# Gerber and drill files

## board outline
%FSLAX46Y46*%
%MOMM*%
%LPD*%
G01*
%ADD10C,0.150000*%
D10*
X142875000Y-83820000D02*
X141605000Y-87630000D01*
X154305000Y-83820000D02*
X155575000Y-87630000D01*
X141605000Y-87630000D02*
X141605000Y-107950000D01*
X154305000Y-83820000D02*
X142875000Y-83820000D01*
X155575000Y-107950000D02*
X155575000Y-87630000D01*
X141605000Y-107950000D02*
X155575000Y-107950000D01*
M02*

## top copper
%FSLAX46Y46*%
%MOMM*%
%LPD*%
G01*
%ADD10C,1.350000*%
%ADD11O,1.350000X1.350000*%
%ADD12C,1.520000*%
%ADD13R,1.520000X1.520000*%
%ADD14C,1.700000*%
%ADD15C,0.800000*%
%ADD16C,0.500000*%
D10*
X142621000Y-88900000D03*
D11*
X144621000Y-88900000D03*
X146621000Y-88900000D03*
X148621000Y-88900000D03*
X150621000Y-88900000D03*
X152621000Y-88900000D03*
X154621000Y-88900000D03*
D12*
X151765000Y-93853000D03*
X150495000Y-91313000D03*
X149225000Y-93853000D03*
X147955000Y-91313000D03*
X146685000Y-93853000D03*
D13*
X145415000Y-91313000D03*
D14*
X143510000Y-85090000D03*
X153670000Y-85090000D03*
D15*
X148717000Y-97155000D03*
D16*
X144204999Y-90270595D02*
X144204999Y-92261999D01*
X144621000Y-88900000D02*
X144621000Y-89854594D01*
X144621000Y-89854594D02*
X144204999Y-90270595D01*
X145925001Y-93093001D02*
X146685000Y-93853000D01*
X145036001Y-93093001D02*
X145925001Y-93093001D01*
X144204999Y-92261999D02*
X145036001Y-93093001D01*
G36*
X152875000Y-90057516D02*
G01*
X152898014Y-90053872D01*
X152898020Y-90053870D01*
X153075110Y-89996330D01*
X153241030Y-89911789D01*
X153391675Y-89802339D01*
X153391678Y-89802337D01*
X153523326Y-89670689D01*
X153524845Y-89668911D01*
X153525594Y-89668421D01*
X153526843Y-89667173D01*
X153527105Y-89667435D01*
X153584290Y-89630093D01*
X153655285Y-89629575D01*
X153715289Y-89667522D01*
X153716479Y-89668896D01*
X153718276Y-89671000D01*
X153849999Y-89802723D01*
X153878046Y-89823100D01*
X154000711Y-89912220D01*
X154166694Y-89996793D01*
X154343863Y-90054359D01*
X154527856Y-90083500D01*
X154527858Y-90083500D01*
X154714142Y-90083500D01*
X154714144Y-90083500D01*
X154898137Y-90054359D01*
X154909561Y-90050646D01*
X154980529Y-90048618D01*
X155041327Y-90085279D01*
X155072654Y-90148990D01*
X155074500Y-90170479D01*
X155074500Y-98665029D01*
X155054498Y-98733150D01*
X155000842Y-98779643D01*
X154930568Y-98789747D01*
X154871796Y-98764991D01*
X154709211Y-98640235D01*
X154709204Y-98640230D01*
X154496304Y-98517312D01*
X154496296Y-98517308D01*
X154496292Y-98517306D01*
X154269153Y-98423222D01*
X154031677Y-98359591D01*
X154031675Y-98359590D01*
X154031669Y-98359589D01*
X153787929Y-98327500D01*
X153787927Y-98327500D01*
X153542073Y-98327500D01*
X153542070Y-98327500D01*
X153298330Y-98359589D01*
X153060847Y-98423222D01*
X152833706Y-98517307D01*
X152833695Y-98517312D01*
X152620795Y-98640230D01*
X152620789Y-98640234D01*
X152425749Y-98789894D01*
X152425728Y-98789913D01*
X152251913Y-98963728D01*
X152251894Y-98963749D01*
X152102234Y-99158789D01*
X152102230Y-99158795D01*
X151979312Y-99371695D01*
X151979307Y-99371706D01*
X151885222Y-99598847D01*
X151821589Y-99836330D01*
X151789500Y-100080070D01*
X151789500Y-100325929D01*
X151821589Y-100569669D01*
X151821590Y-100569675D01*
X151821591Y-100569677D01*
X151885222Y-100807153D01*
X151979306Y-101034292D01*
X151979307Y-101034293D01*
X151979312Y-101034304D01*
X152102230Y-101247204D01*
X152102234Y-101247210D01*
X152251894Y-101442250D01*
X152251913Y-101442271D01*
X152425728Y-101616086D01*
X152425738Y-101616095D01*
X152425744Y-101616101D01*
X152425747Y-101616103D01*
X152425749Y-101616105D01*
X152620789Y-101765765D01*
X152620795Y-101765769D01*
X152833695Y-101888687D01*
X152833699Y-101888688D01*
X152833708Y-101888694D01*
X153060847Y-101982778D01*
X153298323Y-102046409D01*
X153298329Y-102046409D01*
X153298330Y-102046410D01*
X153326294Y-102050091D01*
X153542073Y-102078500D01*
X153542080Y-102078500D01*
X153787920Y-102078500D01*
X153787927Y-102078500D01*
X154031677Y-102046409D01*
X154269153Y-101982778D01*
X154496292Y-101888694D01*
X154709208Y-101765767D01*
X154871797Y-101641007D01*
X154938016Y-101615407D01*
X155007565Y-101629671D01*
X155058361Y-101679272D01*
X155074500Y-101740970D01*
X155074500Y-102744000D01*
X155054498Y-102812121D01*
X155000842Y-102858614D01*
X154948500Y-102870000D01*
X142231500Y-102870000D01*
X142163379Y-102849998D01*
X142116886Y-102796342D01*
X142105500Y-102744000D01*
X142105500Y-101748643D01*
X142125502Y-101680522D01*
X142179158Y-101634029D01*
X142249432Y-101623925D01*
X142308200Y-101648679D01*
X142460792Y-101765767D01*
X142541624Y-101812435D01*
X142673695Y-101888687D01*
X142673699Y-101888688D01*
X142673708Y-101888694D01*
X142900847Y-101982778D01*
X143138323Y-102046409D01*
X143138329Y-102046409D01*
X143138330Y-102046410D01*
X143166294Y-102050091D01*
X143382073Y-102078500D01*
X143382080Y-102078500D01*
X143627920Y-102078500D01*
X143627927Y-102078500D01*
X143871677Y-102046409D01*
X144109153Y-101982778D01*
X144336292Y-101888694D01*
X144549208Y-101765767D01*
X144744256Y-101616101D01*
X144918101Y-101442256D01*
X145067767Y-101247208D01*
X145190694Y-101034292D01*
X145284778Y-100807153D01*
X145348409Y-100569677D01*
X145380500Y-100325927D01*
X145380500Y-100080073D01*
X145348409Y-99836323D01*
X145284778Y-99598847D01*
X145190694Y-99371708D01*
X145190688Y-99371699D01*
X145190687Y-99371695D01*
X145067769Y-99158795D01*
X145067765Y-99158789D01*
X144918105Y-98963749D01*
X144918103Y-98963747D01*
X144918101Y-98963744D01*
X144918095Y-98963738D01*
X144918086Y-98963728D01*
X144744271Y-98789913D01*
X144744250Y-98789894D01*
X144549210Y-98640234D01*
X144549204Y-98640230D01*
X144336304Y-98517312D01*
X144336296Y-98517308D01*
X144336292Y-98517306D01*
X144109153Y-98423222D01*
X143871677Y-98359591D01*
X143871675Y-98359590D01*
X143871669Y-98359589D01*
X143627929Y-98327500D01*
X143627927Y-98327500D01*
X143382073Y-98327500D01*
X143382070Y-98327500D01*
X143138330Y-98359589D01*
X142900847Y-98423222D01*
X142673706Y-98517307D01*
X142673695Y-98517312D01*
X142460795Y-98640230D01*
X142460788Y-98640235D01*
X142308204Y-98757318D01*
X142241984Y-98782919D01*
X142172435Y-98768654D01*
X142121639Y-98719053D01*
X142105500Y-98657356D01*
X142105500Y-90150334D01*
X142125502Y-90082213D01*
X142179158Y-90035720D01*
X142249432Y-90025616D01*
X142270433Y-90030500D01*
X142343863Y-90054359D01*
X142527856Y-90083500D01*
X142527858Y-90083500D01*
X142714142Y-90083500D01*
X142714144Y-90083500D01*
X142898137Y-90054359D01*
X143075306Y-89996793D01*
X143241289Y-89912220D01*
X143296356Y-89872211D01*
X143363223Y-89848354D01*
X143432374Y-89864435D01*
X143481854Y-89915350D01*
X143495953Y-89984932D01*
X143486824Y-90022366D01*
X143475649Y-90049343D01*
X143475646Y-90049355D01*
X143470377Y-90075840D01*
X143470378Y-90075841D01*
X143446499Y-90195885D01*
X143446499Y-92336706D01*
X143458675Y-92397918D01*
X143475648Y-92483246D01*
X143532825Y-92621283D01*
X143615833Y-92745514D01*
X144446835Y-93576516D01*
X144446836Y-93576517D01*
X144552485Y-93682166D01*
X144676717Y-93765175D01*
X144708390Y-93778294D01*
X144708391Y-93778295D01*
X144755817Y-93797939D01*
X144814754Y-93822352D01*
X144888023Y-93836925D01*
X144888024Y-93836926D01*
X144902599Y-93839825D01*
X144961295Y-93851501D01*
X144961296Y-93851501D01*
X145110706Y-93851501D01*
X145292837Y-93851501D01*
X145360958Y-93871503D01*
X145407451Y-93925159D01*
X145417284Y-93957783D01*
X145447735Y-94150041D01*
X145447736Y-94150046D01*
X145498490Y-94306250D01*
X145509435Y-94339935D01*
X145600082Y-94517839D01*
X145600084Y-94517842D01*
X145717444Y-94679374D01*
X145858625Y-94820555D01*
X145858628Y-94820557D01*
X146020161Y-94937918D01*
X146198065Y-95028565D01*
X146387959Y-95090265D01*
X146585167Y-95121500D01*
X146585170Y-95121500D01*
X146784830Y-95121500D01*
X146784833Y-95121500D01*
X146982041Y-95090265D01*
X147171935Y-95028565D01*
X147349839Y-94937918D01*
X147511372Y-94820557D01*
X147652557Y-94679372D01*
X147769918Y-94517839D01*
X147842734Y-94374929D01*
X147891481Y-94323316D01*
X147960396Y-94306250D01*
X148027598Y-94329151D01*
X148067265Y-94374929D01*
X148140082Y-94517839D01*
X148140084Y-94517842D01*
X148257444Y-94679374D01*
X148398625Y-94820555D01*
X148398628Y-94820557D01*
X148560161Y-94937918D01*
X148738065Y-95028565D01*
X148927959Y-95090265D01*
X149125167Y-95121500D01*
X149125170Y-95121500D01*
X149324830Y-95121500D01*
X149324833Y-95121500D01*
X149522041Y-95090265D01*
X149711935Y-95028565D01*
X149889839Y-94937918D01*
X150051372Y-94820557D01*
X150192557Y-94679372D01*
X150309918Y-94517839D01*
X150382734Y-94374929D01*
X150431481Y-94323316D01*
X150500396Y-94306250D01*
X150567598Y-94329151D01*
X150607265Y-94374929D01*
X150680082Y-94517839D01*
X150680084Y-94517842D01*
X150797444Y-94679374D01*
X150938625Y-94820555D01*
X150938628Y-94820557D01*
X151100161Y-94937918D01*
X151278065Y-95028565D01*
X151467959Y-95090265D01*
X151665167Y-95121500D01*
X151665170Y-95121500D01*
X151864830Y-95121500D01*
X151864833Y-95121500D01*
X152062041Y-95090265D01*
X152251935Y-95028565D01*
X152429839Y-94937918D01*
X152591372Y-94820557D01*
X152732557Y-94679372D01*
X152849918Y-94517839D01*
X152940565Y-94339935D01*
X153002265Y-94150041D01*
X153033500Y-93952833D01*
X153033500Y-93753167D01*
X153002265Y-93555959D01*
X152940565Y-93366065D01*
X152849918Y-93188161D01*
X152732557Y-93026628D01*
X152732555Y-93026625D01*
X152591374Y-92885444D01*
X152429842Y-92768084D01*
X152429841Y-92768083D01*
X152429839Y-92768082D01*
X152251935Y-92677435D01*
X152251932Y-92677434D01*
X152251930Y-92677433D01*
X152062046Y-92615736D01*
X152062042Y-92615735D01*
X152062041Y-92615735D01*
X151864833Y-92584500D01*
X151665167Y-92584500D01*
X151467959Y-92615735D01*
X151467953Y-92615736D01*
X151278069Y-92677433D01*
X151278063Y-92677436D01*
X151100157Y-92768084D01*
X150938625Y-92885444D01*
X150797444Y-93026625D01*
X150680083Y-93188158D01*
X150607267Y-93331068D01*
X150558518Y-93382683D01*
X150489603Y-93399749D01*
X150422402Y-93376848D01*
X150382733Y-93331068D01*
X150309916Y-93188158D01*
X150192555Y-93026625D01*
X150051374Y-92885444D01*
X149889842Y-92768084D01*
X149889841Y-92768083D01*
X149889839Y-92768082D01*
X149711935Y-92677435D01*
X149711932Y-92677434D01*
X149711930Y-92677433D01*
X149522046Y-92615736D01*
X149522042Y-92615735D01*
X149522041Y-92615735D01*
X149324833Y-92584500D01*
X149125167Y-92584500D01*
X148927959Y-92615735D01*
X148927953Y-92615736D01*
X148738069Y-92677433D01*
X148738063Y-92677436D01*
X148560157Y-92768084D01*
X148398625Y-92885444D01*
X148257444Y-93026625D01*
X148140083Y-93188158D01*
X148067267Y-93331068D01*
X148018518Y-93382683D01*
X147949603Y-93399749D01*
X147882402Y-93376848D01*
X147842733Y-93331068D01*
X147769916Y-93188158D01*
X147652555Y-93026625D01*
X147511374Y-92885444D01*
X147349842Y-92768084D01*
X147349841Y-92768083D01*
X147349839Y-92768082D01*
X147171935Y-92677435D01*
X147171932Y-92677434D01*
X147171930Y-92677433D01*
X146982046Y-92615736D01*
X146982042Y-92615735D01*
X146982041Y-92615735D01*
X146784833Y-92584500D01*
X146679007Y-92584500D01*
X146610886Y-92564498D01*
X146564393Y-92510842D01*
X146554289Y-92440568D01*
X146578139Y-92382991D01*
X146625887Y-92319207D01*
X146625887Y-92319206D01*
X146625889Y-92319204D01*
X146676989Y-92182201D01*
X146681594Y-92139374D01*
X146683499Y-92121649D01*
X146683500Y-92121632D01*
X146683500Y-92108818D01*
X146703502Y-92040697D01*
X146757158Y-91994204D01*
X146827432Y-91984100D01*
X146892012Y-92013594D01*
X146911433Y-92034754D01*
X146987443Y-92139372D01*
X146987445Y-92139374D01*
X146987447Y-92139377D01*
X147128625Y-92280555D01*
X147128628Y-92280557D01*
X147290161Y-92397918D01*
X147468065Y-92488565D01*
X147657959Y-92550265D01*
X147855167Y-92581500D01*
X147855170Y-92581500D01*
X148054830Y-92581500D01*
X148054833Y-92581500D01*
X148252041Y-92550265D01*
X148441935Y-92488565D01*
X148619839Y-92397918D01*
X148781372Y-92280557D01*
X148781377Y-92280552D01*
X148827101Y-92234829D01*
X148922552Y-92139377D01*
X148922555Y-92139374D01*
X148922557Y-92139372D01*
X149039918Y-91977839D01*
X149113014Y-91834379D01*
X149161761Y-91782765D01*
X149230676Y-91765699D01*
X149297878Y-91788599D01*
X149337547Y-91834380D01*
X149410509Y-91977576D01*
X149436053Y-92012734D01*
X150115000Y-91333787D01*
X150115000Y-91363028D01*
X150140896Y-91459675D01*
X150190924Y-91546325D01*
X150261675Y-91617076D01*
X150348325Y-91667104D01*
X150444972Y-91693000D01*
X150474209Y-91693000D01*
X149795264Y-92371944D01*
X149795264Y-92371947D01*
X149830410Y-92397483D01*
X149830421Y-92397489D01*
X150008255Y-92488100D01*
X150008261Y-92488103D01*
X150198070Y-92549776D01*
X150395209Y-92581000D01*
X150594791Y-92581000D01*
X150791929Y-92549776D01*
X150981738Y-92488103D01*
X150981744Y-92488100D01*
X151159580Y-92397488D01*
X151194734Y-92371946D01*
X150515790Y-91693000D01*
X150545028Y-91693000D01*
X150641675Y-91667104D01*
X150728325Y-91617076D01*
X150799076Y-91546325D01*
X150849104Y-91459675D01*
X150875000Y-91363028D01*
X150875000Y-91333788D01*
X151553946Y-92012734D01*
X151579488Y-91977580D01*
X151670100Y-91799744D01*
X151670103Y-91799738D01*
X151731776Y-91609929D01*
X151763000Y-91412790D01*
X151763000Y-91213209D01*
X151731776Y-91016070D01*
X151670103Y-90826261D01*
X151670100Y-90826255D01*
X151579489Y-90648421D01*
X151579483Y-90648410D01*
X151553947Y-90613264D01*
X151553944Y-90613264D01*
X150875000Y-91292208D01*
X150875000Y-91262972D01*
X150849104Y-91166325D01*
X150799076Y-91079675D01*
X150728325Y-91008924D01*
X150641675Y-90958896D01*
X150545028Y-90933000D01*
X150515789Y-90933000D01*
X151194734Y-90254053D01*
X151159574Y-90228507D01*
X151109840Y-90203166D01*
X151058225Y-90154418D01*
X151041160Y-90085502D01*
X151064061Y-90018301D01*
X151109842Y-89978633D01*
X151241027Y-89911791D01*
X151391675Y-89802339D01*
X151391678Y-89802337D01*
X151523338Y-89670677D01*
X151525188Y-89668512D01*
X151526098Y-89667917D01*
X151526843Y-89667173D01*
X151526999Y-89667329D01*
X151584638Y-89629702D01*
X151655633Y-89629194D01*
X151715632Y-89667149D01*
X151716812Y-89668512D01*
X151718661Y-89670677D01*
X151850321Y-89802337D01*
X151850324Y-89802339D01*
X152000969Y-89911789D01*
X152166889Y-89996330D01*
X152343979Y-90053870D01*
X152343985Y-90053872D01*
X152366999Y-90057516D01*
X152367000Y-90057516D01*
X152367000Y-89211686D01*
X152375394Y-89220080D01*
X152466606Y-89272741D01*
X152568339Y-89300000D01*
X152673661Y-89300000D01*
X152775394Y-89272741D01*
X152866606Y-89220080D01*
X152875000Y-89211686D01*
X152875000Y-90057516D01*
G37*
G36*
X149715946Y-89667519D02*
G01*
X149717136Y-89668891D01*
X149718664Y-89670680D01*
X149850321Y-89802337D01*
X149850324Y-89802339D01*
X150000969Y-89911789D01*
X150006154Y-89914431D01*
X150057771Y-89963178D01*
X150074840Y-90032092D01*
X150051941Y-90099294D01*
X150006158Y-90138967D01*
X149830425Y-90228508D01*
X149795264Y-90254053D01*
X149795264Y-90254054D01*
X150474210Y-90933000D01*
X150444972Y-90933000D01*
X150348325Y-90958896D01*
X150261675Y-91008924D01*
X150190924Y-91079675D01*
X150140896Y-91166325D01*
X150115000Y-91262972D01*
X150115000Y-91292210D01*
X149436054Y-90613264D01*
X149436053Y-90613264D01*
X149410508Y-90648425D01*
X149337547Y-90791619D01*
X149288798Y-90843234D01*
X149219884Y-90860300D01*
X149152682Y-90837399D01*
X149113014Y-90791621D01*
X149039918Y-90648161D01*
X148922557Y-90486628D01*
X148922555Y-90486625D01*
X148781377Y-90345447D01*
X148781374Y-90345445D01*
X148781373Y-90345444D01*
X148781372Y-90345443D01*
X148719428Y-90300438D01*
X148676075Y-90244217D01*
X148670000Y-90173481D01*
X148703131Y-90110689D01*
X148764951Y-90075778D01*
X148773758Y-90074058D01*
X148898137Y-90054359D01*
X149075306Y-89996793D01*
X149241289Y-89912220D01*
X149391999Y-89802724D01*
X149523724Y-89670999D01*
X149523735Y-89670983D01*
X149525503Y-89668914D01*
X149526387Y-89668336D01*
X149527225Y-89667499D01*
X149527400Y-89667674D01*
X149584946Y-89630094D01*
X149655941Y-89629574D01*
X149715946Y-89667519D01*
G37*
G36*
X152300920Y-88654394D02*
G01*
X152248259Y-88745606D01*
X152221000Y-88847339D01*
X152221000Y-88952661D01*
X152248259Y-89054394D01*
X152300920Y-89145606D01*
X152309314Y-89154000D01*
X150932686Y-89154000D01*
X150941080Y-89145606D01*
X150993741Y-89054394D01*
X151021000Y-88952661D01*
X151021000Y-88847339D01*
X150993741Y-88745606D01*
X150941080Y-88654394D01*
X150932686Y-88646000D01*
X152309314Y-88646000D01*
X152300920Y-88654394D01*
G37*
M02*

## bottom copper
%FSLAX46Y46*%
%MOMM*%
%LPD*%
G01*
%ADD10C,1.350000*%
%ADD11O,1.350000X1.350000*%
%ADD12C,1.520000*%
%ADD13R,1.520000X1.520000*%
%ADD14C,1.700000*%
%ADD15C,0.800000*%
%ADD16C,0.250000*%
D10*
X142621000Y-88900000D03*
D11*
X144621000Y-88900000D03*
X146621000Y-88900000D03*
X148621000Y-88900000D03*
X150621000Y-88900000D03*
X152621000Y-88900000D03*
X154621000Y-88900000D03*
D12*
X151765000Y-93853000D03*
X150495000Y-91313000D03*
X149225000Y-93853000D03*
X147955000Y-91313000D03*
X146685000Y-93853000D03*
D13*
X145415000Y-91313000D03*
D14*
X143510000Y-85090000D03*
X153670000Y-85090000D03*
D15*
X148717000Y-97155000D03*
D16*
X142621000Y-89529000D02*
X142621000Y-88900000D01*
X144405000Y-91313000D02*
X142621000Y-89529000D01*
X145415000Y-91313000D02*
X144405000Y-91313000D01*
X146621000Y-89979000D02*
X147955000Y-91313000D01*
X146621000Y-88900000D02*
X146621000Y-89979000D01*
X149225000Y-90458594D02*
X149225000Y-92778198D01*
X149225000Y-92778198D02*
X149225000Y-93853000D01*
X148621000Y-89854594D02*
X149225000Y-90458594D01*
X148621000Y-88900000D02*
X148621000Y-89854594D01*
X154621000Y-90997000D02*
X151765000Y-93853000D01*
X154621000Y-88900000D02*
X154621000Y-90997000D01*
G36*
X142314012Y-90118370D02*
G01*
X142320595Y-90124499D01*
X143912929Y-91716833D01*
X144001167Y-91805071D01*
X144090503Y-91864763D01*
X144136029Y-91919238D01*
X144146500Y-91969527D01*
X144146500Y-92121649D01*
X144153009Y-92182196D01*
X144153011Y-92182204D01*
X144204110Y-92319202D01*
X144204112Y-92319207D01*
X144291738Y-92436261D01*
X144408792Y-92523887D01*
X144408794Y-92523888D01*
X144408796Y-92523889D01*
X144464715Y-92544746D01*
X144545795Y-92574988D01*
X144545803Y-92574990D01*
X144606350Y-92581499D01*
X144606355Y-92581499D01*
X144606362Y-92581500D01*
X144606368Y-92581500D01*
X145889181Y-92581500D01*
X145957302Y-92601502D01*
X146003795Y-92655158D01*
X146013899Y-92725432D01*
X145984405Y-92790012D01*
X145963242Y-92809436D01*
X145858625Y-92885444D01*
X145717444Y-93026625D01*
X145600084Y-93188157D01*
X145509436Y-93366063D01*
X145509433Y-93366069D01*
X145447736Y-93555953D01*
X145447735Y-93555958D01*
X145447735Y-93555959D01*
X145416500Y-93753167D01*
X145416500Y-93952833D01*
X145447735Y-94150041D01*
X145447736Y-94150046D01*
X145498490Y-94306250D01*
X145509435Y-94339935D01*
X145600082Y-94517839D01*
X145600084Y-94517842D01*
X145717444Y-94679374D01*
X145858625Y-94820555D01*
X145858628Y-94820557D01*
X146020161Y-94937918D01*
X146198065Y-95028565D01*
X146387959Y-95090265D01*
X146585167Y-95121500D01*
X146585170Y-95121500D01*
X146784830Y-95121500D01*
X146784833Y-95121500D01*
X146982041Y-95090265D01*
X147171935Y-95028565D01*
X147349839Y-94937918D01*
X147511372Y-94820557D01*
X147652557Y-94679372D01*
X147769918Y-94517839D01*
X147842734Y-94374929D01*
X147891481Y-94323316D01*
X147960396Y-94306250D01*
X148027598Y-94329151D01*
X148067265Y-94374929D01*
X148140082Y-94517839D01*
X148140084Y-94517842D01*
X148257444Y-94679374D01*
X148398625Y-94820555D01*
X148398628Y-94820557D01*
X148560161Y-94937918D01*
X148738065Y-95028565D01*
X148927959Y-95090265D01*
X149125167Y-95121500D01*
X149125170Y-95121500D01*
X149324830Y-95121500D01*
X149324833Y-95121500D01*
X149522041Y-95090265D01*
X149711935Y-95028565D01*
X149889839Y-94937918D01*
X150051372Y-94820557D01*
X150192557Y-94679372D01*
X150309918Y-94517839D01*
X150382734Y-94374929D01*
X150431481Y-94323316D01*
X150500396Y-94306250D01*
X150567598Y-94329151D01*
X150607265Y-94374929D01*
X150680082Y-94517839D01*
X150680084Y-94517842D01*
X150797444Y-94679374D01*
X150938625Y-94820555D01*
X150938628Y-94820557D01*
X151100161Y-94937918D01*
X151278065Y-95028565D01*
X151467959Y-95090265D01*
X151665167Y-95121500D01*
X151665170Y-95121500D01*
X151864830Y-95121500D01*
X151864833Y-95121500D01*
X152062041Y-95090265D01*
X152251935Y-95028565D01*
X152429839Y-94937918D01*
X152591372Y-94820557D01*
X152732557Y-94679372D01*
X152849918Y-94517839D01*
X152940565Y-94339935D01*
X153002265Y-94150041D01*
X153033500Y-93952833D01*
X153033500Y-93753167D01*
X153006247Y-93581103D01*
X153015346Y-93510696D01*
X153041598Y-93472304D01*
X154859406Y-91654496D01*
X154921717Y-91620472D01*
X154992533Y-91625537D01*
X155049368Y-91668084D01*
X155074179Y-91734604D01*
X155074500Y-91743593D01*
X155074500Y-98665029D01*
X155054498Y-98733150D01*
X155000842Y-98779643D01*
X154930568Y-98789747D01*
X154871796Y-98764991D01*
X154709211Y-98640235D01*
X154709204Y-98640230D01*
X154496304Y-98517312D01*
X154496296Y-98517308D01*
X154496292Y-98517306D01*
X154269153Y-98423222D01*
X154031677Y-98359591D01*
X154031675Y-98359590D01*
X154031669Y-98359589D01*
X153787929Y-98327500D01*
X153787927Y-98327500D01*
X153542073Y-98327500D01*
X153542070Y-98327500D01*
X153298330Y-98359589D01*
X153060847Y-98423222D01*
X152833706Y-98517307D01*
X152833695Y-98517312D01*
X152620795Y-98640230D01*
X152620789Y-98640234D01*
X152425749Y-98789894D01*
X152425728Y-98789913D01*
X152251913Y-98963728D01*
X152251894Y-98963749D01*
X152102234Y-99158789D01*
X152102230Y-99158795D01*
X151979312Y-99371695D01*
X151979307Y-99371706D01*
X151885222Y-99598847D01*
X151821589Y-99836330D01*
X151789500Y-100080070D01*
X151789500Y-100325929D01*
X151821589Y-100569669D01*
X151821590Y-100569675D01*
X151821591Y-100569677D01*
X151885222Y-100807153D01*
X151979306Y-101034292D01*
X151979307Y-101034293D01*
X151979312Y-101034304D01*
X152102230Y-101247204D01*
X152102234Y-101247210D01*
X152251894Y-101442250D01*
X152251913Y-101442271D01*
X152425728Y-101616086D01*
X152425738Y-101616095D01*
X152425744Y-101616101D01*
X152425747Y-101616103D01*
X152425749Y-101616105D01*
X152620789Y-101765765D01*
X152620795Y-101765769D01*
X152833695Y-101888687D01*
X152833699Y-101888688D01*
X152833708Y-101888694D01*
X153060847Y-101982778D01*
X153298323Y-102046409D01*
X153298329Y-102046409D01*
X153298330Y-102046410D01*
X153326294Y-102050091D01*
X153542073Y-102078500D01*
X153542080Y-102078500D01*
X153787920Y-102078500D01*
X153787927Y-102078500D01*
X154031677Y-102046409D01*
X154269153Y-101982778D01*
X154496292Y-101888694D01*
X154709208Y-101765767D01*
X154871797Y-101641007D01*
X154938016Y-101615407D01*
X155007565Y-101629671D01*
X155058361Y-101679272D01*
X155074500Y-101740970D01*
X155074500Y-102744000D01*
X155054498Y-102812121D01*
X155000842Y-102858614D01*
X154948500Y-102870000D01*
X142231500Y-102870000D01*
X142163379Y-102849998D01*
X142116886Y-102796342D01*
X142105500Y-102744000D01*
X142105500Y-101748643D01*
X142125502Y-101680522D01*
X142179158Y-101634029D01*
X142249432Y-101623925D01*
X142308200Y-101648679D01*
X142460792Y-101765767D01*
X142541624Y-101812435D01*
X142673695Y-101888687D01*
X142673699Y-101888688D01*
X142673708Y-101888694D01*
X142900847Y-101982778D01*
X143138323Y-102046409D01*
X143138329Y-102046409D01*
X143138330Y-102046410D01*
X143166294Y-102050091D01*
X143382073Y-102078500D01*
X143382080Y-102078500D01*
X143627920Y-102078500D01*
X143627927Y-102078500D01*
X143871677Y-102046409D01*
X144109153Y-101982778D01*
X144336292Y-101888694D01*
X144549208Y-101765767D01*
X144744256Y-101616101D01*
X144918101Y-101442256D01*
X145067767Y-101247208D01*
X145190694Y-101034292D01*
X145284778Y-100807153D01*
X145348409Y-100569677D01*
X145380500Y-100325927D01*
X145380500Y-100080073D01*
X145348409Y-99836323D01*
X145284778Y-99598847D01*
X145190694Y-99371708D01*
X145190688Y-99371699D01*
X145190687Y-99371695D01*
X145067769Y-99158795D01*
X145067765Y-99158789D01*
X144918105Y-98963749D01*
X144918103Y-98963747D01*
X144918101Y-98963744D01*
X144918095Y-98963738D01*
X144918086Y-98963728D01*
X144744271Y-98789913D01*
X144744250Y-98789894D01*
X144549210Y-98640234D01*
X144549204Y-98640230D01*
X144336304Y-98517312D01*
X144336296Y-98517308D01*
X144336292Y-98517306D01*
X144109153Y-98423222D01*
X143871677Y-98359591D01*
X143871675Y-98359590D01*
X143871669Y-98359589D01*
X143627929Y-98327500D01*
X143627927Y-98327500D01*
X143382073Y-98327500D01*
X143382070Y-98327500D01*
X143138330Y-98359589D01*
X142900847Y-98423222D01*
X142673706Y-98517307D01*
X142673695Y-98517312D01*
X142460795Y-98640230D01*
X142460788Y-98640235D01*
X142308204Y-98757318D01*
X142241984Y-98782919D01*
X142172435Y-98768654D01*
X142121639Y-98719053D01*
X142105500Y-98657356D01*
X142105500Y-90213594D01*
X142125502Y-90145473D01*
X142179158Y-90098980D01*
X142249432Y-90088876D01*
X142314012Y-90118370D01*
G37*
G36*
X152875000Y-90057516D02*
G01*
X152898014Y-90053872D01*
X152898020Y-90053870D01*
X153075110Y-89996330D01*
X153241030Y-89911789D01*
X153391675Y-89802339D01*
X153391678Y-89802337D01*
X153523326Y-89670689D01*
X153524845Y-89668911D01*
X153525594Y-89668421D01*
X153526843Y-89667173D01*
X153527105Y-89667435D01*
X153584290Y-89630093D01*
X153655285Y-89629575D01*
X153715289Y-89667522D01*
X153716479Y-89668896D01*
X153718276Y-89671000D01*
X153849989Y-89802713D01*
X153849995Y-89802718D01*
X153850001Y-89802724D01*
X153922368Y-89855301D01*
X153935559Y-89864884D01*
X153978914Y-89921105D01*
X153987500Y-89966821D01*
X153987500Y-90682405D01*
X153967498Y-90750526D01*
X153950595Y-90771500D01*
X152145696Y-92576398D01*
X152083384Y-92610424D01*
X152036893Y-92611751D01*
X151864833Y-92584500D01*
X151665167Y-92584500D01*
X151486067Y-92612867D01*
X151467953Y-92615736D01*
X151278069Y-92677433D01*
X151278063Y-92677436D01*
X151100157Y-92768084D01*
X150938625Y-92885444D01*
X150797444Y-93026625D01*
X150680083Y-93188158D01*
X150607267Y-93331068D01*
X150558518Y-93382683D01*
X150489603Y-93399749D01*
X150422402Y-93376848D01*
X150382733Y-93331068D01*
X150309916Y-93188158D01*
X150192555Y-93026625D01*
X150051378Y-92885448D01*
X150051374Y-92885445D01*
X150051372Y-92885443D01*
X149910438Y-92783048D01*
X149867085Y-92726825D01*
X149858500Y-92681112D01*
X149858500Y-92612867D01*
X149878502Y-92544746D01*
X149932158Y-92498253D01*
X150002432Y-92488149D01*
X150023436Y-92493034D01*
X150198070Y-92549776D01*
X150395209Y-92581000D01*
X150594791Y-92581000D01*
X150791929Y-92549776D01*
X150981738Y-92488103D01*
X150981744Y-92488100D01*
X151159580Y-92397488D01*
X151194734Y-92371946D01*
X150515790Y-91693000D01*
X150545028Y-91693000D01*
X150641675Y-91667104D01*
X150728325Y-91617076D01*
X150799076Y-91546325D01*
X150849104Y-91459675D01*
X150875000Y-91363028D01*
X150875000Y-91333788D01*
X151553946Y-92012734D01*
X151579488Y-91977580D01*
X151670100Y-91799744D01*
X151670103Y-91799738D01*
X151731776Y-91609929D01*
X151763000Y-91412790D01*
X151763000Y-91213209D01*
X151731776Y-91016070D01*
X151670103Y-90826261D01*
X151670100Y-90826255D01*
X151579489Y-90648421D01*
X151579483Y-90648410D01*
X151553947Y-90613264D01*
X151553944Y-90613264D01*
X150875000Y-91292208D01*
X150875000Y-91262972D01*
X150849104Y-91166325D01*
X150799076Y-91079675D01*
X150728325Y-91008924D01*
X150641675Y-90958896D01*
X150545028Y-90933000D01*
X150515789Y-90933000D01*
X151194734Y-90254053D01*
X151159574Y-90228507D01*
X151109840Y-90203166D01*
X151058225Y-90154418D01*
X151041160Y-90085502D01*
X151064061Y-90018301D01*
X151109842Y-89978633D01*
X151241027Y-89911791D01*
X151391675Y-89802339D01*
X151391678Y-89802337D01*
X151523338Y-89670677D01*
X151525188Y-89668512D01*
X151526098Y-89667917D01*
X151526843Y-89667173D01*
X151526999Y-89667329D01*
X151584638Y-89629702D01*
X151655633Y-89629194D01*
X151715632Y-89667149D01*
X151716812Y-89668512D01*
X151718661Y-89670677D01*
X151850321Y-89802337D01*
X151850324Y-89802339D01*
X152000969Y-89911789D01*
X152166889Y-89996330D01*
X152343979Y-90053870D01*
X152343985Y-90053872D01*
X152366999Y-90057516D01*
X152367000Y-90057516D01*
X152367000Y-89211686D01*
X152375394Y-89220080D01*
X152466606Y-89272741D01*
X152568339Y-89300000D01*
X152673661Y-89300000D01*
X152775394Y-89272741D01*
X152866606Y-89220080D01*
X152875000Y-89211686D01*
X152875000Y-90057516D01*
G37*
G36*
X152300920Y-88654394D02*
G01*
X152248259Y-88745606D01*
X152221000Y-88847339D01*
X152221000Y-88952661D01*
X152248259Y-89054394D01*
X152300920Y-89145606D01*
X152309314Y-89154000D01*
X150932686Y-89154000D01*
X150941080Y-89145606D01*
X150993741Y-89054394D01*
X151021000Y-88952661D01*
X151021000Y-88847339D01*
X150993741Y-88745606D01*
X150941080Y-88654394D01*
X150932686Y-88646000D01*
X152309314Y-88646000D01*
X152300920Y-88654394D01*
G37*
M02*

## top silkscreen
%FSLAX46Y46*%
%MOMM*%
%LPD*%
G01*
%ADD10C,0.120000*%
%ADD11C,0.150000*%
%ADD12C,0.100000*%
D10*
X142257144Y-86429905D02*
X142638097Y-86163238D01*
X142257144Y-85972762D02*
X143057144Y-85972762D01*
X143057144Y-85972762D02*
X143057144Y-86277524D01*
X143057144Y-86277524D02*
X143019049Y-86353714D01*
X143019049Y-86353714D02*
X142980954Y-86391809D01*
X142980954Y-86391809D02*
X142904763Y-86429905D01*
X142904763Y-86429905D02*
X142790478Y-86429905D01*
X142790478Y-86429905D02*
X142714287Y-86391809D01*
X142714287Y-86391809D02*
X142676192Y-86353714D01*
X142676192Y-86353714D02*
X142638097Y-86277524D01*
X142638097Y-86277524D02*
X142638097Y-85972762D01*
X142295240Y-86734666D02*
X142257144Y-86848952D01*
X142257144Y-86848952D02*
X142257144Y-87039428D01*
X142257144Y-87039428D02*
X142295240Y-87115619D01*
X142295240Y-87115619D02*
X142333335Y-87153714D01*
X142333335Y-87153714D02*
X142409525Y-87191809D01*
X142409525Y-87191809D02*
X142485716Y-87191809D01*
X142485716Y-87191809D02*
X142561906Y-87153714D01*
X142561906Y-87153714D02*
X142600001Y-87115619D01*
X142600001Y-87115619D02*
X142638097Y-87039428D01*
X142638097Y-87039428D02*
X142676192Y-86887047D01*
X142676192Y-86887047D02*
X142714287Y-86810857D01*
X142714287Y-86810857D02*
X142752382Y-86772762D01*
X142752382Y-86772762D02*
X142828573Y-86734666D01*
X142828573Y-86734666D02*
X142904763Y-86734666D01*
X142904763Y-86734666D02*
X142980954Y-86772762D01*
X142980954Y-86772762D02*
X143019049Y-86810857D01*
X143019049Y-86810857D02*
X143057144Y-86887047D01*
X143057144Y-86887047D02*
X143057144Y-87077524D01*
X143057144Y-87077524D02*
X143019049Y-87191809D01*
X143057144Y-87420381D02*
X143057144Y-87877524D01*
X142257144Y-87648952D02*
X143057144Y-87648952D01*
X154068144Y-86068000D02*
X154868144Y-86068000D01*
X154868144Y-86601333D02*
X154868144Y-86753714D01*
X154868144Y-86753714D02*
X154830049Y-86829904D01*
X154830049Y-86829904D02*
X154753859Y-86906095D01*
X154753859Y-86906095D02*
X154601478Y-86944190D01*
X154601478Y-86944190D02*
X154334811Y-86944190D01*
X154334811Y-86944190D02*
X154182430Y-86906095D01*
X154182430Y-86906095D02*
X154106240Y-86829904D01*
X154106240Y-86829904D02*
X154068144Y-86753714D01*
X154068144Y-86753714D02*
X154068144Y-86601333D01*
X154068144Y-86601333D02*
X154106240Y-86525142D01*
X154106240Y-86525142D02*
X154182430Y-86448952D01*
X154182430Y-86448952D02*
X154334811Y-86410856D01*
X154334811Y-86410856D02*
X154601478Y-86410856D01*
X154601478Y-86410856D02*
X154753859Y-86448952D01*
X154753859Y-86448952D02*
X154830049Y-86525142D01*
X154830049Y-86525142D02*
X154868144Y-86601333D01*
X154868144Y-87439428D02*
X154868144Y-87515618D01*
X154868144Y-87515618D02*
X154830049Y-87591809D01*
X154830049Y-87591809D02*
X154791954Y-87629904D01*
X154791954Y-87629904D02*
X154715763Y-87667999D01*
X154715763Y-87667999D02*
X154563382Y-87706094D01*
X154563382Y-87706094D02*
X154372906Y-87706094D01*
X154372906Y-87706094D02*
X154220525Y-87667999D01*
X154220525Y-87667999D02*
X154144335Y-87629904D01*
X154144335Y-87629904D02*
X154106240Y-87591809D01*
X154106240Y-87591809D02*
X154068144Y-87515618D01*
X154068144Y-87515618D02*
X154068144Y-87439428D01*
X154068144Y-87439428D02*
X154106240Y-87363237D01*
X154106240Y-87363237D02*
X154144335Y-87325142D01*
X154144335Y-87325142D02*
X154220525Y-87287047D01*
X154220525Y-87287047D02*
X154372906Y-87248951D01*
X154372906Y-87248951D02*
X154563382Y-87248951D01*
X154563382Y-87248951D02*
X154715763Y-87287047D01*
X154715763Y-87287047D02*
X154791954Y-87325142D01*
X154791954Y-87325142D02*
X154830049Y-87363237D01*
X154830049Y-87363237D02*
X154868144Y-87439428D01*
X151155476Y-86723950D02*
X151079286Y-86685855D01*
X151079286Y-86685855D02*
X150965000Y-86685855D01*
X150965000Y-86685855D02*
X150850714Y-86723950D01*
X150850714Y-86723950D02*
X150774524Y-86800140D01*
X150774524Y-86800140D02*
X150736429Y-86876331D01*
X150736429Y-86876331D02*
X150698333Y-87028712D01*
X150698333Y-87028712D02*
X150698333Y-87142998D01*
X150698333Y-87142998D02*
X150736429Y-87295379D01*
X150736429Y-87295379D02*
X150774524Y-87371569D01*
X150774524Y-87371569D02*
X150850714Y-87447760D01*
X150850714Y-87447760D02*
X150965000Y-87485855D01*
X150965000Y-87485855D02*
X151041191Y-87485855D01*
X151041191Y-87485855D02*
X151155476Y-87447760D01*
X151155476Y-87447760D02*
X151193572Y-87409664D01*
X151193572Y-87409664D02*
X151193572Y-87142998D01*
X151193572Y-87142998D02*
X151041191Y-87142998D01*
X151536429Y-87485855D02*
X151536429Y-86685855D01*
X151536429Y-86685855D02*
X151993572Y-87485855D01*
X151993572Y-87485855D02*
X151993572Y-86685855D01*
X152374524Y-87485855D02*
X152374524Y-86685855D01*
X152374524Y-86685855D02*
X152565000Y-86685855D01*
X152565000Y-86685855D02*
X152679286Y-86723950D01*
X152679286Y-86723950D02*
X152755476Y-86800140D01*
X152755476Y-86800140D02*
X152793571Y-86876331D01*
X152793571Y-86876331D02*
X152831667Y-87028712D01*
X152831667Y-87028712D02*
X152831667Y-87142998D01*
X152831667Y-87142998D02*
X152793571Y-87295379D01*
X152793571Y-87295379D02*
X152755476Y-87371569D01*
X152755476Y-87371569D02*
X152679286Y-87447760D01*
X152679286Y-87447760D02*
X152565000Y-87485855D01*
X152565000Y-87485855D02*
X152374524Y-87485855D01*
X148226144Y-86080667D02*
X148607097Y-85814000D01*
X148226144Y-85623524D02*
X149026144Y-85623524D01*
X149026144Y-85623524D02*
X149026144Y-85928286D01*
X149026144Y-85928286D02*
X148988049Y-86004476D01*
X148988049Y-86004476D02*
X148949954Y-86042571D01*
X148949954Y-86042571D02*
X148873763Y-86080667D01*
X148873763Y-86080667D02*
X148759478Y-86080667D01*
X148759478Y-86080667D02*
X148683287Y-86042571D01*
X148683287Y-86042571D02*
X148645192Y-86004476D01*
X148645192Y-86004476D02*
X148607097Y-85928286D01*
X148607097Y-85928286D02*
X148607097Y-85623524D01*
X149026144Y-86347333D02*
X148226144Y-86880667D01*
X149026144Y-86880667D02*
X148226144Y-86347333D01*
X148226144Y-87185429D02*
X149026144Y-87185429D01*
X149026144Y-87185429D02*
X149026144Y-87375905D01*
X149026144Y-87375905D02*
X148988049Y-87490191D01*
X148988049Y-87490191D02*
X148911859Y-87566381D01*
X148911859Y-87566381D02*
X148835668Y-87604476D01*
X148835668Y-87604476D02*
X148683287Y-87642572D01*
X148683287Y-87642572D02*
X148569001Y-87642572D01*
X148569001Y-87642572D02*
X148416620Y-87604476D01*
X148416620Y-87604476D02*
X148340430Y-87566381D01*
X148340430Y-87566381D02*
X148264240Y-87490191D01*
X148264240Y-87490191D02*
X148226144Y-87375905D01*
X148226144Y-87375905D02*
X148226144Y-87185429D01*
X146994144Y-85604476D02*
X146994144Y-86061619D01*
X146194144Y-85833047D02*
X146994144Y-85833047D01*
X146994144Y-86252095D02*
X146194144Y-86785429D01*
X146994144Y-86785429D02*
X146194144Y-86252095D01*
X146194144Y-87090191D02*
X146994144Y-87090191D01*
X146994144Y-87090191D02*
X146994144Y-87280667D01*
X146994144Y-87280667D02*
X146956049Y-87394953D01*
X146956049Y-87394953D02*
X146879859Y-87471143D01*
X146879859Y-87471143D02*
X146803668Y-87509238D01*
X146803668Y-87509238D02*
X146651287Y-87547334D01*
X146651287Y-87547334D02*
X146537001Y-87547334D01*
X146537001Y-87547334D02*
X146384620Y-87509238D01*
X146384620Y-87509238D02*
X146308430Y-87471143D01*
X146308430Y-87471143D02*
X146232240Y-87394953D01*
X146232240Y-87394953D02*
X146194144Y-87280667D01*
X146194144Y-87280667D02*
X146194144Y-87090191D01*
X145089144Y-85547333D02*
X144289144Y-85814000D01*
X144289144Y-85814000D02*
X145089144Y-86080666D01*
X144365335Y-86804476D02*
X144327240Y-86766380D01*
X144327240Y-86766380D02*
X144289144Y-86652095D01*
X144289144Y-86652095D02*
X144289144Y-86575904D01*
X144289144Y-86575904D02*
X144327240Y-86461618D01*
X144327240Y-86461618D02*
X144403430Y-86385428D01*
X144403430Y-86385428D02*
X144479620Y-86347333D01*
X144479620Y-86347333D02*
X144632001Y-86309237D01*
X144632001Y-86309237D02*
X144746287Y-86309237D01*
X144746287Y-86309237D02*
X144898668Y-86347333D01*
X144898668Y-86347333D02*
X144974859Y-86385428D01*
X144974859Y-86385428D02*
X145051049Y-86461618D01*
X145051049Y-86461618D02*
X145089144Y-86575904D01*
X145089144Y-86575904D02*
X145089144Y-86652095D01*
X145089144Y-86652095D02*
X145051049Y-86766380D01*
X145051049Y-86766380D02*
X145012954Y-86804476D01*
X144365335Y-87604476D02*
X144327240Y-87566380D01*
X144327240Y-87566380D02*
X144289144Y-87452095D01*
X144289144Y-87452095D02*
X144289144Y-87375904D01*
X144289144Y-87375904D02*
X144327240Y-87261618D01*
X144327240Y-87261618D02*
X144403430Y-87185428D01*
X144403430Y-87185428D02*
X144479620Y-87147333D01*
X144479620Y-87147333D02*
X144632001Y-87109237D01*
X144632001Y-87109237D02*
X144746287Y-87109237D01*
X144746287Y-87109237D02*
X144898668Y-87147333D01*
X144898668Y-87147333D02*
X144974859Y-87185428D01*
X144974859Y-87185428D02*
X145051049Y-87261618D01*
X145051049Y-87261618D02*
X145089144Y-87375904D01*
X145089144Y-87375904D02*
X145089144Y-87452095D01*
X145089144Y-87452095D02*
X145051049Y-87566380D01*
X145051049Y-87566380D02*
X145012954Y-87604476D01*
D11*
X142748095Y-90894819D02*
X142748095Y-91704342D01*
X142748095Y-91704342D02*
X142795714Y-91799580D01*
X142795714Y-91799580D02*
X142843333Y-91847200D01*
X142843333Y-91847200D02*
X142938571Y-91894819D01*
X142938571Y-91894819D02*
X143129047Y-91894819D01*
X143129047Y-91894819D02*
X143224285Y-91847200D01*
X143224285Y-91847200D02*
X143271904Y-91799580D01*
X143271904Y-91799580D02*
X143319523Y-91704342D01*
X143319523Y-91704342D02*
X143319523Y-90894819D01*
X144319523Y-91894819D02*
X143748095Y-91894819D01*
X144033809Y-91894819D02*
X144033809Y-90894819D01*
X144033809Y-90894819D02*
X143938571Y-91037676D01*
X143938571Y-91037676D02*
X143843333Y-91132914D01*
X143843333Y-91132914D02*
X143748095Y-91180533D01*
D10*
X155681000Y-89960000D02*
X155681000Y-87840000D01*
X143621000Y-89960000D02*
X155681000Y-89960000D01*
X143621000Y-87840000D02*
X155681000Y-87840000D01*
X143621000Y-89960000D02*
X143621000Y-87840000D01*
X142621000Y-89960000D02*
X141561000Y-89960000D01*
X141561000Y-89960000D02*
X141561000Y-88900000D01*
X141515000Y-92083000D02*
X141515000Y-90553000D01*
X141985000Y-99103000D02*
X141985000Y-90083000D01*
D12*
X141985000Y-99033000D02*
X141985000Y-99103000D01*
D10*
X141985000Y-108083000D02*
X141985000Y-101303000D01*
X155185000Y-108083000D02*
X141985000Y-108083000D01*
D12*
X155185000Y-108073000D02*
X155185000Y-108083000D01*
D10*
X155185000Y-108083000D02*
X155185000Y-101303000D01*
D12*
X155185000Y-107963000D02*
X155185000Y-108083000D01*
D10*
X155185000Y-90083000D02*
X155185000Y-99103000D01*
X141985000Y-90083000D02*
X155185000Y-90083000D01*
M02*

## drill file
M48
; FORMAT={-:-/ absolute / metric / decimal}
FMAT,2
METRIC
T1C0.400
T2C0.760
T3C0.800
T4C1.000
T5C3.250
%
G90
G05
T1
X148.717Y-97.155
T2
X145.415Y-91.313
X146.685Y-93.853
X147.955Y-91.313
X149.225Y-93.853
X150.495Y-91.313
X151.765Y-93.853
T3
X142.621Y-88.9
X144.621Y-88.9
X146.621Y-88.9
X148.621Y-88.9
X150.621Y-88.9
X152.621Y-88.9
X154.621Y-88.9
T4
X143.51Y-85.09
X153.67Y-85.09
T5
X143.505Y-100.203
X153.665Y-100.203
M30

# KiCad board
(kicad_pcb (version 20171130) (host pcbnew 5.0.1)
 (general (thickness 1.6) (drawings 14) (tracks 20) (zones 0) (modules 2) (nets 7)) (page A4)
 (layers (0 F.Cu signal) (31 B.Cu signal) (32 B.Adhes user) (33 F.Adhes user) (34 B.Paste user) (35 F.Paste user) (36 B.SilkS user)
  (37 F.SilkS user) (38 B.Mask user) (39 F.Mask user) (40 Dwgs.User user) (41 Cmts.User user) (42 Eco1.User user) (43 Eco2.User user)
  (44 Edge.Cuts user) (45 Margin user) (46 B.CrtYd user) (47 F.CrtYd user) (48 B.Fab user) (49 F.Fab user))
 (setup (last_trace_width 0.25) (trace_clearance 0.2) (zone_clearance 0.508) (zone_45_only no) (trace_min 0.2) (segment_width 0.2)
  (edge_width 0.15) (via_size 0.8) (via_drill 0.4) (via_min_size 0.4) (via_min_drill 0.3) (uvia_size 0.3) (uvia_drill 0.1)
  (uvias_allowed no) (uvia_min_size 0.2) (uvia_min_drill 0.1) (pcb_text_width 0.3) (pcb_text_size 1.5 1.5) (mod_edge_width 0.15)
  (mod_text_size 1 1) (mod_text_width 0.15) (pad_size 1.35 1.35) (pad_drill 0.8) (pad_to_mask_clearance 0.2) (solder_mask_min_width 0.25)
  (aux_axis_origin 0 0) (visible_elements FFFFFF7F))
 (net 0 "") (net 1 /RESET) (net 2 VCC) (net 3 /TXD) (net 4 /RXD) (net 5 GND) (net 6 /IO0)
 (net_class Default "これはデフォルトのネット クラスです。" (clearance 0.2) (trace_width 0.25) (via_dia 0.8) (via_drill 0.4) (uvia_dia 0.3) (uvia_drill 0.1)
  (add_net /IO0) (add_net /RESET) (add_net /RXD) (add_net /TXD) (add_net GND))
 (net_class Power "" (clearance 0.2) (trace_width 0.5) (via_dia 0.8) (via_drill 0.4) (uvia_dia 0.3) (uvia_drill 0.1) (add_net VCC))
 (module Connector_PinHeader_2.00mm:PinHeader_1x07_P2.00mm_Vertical (layer F.Cu) (at 142.621 88.9 90)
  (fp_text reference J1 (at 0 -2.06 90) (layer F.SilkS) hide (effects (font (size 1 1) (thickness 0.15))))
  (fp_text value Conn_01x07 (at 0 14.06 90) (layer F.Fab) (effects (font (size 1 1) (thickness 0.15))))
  (fp_line (start -1.06 13.06) (end 1.06 13.06) (layer F.SilkS) (width 0.12))
  (fp_line (start -1.06 1) (end -1.06 13.06) (layer F.SilkS) (width 0.12))
  (fp_line (start 1.06 1) (end 1.06 13.06) (layer F.SilkS) (width 0.12))
  (fp_line (start -1.06 1) (end 1.06 1) (layer F.SilkS) (width 0.12))
  (fp_line (start -1.06 0) (end -1.06 -1.06) (layer F.SilkS) (width 0.12))
  (fp_line (start -1.06 -1.06) (end 0 -1.06) (layer F.SilkS) (width 0.12))
  (pad 1 thru_hole circle (at 0 0 90) (size 1.35 1.35) (drill 0.8) (layers *.Cu *.Mask) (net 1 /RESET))
  (pad 2 thru_hole oval (at 0 2 90) (size 1.35 1.35) (drill 0.8) (layers *.Cu *.Mask) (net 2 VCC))
  (pad 3 thru_hole oval (at 0 4 90) (size 1.35 1.35) (drill 0.8) (layers *.Cu *.Mask) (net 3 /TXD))
  (pad 4 thru_hole oval (at 0 6 90) (size 1.35 1.35) (drill 0.8) (layers *.Cu *.Mask) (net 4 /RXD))
  (pad 5 thru_hole oval (at 0 8 90) (size 1.35 1.35) (drill 0.8) (layers *.Cu *.Mask) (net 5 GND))
  (pad 6 thru_hole oval (at 0 10 90) (size 1.35 1.35) (drill 0.8) (layers *.Cu *.Mask) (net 5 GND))
  (pad 7 thru_hole oval (at 0 12 90) (size 1.35 1.35) (drill 0.8) (layers *.Cu *.Mask) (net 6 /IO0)))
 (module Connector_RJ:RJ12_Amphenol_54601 (layer F.Cu) (at 145.415 91.313)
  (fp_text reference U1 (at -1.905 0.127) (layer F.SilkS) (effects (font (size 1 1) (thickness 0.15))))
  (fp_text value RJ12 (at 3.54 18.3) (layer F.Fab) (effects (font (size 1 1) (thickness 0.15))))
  (fp_line (start -3.9 0.77) (end -3.9 -0.76) (layer F.SilkS) (width 0.12))
  (fp_line (start -3.43 7.79) (end -3.43 -1.23) (layer F.SilkS) (width 0.12))
  (fp_line (start -3.43 7.72) (end -3.43 7.79) (layer F.SilkS) (width 0.1))
  (fp_line (start -3.43 16.77) (end -3.43 9.99) (layer F.SilkS) (width 0.12))
  (fp_line (start 9.77 16.77) (end -3.43 16.77) (layer F.SilkS) (width 0.12))
  (fp_line (start 9.77 16.76) (end 9.77 16.77) (layer F.SilkS) (width 0.1))
  (fp_line (start 9.77 16.77) (end 9.77 9.99) (layer F.SilkS) (width 0.12))
  (fp_line (start 9.77 16.65) (end 9.77 16.77) (layer F.SilkS) (width 0.1))
  (fp_line (start 9.77 -1.23) (end 9.77 7.79) (layer F.SilkS) (width 0.12))
  (fp_line (start -3.43 -1.23) (end 9.77 -1.23) (layer F.SilkS) (width 0.12))
  (pad "" np_thru_hole circle (at 8.25 8.89) (size 3.25 3.25) (drill 3.25) (layers *.Cu *.Mask))
  (pad 6 thru_hole circle (at 6.35 2.54) (size 1.52 1.52) (drill 0.76) (layers *.Cu *.Mask) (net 6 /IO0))
  (pad 5 thru_hole circle (at 5.08 0) (size 1.52 1.52) (drill 0.76) (layers *.Cu *.Mask) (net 5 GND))
  (pad 4 thru_hole circle (at 3.81 2.54) (size 1.52 1.52) (drill 0.76) (layers *.Cu *.Mask) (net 4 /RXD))
  (pad 3 thru_hole circle (at 2.54 0) (size 1.52 1.52) (drill 0.76) (layers *.Cu *.Mask) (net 3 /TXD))
  (pad 2 thru_hole circle (at 1.27 2.54) (size 1.52 1.52) (drill 0.76) (layers *.Cu *.Mask) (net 2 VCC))
  (pad "" np_thru_hole circle (at -1.91 8.89) (size 3.25 3.25) (drill 3.25) (layers *.Cu *.Mask))
  (pad 1 thru_hole rect (at 0 0) (size 1.52 1.52) (drill 0.76) (layers *.Cu *.Mask) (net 1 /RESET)))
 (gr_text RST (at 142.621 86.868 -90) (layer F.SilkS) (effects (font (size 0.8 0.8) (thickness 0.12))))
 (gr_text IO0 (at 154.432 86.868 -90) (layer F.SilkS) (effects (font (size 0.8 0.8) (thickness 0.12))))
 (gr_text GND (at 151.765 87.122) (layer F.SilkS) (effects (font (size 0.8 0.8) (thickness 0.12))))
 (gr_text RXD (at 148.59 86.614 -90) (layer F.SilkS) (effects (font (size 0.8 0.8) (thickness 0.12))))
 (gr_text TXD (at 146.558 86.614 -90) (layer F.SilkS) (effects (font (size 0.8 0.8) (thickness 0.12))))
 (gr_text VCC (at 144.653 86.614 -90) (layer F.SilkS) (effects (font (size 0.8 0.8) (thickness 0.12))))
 (gr_line (start 142.875 83.82) (end 141.605 87.63) (layer Edge.Cuts) (width 0.15))
 (gr_line (start 154.305 83.82) (end 155.575 87.63) (layer Edge.Cuts) (width 0.15))
 (gr_line (start 141.605 87.63) (end 141.605 107.95) (layer Edge.Cuts) (width 0.15))
 (gr_line (start 154.305 83.82) (end 142.875 83.82) (layer Edge.Cuts) (width 0.15))
 (gr_line (start 155.575 107.95) (end 155.575 87.63) (layer Edge.Cuts) (width 0.15))
 (gr_line (start 141.605 107.95) (end 155.575 107.95) (layer Edge.Cuts) (width 0.15))
 (via (at 143.51 85.09) (size 1.7) (drill 1) (layers F.Cu B.Cu) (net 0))
 (via (at 153.67 85.09) (size 1.7) (drill 1) (layers F.Cu B.Cu) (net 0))
 (segment (start 144.204999 90.270595) (end 144.204999 92.261999) (width 0.5) (layer F.Cu) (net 2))
 (segment (start 144.621 88.9) (end 144.621 89.854594) (width 0.5) (layer F.Cu) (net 2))
 (segment (start 144.621 89.854594) (end 144.204999 90.270595) (width 0.5) (layer F.Cu) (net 2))
 (segment (start 145.925001 93.093001) (end 146.685 93.853) (width 0.5) (layer F.Cu) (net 2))
 (segment (start 145.036001 93.093001) (end 145.925001 93.093001) (width 0.5) (layer F.Cu) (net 2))
 (segment (start 144.204999 92.261999) (end 145.036001 93.093001) (width 0.5) (layer F.Cu) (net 2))
 (via (at 148.717 97.155) (size 0.8) (drill 0.4) (layers F.Cu B.Cu) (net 5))
 (segment (start 142.621 89.529) (end 142.621 88.9) (width 0.25) (layer B.Cu) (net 1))
 (segment (start 144.405 91.313) (end 142.621 89.529) (width 0.25) (layer B.Cu) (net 1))
 (segment (start 145.415 91.313) (end 144.405 91.313) (width 0.25) (layer B.Cu) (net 1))
 (segment (start 146.621 89.979) (end 147.955 91.313) (width 0.25) (layer B.Cu) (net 3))
 (segment (start 146.621 88.9) (end 146.621 89.979) (width 0.25) (layer B.Cu) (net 3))
 (segment (start 149.225 90.458594) (end 149.225 92.778198) (width 0.25) (layer B.Cu) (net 4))
 (segment (start 149.225 92.778198) (end 149.225 93.853) (width 0.25) (layer B.Cu) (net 4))
 (segment (start 148.621 89.854594) (end 149.225 90.458594) (width 0.25) (layer B.Cu) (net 4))
 (segment (start 148.621 88.9) (end 148.621 89.854594) (width 0.25) (layer B.Cu) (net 4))
 (segment (start 154.621 90.997) (end 151.765 93.853) (width 0.25) (layer B.Cu) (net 6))
 (segment (start 154.621 88.9) (end 154.621 90.997) (width 0.25) (layer B.Cu) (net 6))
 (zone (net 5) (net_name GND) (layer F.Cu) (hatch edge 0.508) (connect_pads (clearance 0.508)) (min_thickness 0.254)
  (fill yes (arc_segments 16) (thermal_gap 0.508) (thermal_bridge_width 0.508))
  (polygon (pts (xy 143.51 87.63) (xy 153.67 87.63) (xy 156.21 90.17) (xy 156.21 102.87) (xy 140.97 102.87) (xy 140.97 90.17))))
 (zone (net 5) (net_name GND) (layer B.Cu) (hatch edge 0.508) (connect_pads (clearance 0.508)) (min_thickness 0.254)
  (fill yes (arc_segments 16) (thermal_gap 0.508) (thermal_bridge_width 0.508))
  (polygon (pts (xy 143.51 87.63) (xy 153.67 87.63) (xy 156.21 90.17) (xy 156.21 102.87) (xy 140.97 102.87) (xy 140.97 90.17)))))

